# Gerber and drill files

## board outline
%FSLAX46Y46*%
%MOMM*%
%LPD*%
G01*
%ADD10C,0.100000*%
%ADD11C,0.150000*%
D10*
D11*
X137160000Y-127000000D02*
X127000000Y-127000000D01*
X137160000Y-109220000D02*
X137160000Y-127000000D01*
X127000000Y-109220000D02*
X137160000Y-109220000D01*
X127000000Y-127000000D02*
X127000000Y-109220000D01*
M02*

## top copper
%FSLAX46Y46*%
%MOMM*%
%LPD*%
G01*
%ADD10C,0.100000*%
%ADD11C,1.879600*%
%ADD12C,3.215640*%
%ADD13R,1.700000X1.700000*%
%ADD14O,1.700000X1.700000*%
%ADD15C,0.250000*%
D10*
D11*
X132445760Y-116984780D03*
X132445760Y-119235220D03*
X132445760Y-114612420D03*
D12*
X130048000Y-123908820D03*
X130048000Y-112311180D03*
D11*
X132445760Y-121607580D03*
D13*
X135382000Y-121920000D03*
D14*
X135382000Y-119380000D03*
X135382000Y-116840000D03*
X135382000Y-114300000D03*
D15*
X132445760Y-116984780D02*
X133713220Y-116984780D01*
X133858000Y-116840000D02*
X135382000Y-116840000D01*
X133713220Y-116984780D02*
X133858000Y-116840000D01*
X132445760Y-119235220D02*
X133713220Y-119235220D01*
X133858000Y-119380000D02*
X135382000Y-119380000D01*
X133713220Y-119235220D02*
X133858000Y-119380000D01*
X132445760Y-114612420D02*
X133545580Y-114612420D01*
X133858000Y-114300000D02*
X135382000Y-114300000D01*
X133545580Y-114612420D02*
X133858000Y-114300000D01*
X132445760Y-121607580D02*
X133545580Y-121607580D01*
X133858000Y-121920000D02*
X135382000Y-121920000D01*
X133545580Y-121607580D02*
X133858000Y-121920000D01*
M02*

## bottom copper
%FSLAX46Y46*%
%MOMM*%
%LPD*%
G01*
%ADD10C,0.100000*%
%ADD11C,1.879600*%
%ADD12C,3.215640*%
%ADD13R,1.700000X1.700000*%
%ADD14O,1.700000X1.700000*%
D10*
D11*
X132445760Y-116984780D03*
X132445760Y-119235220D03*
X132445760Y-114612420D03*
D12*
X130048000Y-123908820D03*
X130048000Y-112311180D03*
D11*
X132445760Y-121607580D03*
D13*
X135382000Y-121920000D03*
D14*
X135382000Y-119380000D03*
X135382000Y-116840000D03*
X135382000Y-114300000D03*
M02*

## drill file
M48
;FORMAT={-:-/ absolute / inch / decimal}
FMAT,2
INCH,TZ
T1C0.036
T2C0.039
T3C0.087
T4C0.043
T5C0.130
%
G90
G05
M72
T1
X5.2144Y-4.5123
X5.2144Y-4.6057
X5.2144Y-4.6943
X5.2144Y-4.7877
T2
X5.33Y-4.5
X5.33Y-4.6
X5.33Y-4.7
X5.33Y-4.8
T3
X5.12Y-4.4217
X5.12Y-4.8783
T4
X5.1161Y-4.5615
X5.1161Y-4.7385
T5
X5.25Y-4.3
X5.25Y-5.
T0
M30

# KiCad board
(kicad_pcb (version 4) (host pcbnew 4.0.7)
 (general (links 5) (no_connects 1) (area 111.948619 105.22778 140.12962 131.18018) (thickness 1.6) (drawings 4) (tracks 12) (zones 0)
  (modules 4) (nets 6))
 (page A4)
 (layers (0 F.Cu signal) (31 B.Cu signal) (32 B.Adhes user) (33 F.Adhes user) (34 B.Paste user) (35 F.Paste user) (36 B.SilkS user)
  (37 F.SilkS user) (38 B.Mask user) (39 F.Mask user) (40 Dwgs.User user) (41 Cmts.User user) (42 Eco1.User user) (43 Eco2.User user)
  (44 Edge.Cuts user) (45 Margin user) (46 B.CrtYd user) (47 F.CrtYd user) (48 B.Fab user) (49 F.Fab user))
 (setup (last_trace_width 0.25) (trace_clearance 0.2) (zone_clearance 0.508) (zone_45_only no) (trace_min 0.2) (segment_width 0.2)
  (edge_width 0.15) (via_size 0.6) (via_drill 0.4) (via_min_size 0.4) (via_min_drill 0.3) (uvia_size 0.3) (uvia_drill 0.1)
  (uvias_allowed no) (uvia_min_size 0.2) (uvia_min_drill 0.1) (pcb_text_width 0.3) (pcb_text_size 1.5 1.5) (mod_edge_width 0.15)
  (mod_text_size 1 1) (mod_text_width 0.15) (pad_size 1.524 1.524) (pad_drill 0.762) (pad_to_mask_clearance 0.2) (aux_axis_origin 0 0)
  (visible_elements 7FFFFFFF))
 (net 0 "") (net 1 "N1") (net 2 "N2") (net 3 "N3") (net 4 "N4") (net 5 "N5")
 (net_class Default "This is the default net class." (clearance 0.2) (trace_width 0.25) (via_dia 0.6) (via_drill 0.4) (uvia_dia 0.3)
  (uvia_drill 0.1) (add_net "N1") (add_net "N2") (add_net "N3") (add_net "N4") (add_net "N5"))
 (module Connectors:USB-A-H (layer F.Cu) (at 130.048 118.11)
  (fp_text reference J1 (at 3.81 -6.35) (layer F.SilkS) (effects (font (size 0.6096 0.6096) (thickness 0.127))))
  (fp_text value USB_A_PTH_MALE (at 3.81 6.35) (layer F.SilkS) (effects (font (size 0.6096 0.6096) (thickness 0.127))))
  (pad D+ thru_hole circle (at 2.39776 -1.12522) (size 1.8796 1.8796) (drill 0.9144) (layers *.Cu *.Mask) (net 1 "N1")
   (solder_mask_margin 0.1016))
  (pad D- thru_hole circle (at 2.39776 1.12522) (size 1.8796 1.8796) (drill 0.9144) (layers *.Cu *.Mask) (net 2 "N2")
   (solder_mask_margin 0.1016))
  (pad GND thru_hole circle (at 2.39776 -3.49758) (size 1.8796 1.8796) (drill 0.9144) (layers *.Cu *.Mask) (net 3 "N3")
   (solder_mask_margin 0.1016))
  (pad SHLD thru_hole circle (at 0 5.79882) (size 3.21564 3.21564) (drill 2.19964) (layers *.Cu *.Mask) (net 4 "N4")
   (solder_mask_margin 0.1016))
  (pad SHLD thru_hole circle (at 0 -5.79882) (size 3.21564 3.21564) (drill 2.19964) (layers *.Cu *.Mask) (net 4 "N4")
   (solder_mask_margin 0.1016))
  (pad VBUS thru_hole circle (at 2.39776 3.49758) (size 1.8796 1.8796) (drill 0.9144) (layers *.Cu *.Mask) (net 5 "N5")
   (solder_mask_margin 0.1016))
  (pad "" np_thru_hole circle (at -0.09906 -2.2479) (size 1.09982 1.09982) (drill 1.09982) (layers *.Cu *.Mask) (solder_mask_margin 0.1016))
  (pad "" np_thru_hole circle (at -0.09906 2.2479) (size 1.09982 1.09982) (drill 1.09982) (layers *.Cu *.Mask) (solder_mask_margin 0.1016)))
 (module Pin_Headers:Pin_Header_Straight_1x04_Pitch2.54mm (layer F.Cu) (at 135.382 121.92 180)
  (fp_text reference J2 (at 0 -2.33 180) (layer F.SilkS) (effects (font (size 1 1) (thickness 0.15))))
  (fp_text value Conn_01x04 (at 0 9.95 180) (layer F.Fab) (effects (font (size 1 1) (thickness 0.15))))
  (pad 1 thru_hole rect (at 0 0 180) (size 1.7 1.7) (drill 1) (layers *.Cu *.Mask) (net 5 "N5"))
  (pad 2 thru_hole oval (at 0 2.54 180) (size 1.7 1.7) (drill 1) (layers *.Cu *.Mask) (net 2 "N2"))
  (pad 3 thru_hole oval (at 0 5.08 180) (size 1.7 1.7) (drill 1) (layers *.Cu *.Mask) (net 1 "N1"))
  (pad 4 thru_hole oval (at 0 7.62 180) (size 1.7 1.7) (drill 1) (layers *.Cu *.Mask) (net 3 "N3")))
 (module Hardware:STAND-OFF (layer F.Cu) (at 133.35 109.22)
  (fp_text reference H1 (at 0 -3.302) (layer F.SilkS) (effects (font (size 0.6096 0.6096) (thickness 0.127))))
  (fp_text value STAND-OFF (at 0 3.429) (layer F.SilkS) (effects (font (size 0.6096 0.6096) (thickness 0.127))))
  (pad "" np_thru_hole circle (at 0 0) (size 3.302 3.302) (drill 3.302) (layers *.Cu *.Mask) (solder_mask_margin 0.1016)))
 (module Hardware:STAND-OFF (layer F.Cu) (at 133.35 127)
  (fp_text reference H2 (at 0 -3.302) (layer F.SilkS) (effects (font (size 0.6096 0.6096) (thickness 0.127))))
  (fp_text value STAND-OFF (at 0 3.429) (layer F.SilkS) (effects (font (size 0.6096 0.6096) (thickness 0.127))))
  (pad "" np_thru_hole circle (at 0 0) (size 3.302 3.302) (drill 3.302) (layers *.Cu *.Mask) (solder_mask_margin 0.1016)))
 (gr_line (start 137.16 127) (end 127 127) (angle 90) (layer Edge.Cuts) (width 0.15))
 (gr_line (start 137.16 109.22) (end 137.16 127) (angle 90) (layer Edge.Cuts) (width 0.15))
 (gr_line (start 127 109.22) (end 137.16 109.22) (angle 90) (layer Edge.Cuts) (width 0.15))
 (gr_line (start 127 127) (end 127 109.22) (angle 90) (layer Edge.Cuts) (width 0.15))
 (segment (start 132.44576 116.98478) (end 133.71322 116.98478) (width 0.25) (layer F.Cu) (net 1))
 (segment (start 133.858 116.84) (end 135.382 116.84) (width 0.25) (layer F.Cu) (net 1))
 (segment (start 133.71322 116.98478) (end 133.858 116.84) (width 0.25) (layer F.Cu) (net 1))
 (segment (start 132.44576 119.23522) (end 133.71322 119.23522) (width 0.25) (layer F.Cu) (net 2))
 (segment (start 133.858 119.38) (end 135.382 119.38) (width 0.25) (layer F.Cu) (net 2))
 (segment (start 133.71322 119.23522) (end 133.858 119.38) (width 0.25) (layer F.Cu) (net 2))
 (segment (start 132.44576 114.61242) (end 133.54558 114.61242) (width 0.25) (layer F.Cu) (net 3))
 (segment (start 133.858 114.3) (end 135.382 114.3) (width 0.25) (layer F.Cu) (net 3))
 (segment (start 133.54558 114.61242) (end 133.858 114.3) (width 0.25) (layer F.Cu) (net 3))
 (segment (start 132.44576 121.60758) (end 133.54558 121.60758) (width 0.25) (layer F.Cu) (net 5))
 (segment (start 133.858 121.92) (end 135.382 121.92) (width 0.25) (layer F.Cu) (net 5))
 (segment (start 133.54558 121.60758) (end 133.858 121.92) (width 0.25) (layer F.Cu) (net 5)))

